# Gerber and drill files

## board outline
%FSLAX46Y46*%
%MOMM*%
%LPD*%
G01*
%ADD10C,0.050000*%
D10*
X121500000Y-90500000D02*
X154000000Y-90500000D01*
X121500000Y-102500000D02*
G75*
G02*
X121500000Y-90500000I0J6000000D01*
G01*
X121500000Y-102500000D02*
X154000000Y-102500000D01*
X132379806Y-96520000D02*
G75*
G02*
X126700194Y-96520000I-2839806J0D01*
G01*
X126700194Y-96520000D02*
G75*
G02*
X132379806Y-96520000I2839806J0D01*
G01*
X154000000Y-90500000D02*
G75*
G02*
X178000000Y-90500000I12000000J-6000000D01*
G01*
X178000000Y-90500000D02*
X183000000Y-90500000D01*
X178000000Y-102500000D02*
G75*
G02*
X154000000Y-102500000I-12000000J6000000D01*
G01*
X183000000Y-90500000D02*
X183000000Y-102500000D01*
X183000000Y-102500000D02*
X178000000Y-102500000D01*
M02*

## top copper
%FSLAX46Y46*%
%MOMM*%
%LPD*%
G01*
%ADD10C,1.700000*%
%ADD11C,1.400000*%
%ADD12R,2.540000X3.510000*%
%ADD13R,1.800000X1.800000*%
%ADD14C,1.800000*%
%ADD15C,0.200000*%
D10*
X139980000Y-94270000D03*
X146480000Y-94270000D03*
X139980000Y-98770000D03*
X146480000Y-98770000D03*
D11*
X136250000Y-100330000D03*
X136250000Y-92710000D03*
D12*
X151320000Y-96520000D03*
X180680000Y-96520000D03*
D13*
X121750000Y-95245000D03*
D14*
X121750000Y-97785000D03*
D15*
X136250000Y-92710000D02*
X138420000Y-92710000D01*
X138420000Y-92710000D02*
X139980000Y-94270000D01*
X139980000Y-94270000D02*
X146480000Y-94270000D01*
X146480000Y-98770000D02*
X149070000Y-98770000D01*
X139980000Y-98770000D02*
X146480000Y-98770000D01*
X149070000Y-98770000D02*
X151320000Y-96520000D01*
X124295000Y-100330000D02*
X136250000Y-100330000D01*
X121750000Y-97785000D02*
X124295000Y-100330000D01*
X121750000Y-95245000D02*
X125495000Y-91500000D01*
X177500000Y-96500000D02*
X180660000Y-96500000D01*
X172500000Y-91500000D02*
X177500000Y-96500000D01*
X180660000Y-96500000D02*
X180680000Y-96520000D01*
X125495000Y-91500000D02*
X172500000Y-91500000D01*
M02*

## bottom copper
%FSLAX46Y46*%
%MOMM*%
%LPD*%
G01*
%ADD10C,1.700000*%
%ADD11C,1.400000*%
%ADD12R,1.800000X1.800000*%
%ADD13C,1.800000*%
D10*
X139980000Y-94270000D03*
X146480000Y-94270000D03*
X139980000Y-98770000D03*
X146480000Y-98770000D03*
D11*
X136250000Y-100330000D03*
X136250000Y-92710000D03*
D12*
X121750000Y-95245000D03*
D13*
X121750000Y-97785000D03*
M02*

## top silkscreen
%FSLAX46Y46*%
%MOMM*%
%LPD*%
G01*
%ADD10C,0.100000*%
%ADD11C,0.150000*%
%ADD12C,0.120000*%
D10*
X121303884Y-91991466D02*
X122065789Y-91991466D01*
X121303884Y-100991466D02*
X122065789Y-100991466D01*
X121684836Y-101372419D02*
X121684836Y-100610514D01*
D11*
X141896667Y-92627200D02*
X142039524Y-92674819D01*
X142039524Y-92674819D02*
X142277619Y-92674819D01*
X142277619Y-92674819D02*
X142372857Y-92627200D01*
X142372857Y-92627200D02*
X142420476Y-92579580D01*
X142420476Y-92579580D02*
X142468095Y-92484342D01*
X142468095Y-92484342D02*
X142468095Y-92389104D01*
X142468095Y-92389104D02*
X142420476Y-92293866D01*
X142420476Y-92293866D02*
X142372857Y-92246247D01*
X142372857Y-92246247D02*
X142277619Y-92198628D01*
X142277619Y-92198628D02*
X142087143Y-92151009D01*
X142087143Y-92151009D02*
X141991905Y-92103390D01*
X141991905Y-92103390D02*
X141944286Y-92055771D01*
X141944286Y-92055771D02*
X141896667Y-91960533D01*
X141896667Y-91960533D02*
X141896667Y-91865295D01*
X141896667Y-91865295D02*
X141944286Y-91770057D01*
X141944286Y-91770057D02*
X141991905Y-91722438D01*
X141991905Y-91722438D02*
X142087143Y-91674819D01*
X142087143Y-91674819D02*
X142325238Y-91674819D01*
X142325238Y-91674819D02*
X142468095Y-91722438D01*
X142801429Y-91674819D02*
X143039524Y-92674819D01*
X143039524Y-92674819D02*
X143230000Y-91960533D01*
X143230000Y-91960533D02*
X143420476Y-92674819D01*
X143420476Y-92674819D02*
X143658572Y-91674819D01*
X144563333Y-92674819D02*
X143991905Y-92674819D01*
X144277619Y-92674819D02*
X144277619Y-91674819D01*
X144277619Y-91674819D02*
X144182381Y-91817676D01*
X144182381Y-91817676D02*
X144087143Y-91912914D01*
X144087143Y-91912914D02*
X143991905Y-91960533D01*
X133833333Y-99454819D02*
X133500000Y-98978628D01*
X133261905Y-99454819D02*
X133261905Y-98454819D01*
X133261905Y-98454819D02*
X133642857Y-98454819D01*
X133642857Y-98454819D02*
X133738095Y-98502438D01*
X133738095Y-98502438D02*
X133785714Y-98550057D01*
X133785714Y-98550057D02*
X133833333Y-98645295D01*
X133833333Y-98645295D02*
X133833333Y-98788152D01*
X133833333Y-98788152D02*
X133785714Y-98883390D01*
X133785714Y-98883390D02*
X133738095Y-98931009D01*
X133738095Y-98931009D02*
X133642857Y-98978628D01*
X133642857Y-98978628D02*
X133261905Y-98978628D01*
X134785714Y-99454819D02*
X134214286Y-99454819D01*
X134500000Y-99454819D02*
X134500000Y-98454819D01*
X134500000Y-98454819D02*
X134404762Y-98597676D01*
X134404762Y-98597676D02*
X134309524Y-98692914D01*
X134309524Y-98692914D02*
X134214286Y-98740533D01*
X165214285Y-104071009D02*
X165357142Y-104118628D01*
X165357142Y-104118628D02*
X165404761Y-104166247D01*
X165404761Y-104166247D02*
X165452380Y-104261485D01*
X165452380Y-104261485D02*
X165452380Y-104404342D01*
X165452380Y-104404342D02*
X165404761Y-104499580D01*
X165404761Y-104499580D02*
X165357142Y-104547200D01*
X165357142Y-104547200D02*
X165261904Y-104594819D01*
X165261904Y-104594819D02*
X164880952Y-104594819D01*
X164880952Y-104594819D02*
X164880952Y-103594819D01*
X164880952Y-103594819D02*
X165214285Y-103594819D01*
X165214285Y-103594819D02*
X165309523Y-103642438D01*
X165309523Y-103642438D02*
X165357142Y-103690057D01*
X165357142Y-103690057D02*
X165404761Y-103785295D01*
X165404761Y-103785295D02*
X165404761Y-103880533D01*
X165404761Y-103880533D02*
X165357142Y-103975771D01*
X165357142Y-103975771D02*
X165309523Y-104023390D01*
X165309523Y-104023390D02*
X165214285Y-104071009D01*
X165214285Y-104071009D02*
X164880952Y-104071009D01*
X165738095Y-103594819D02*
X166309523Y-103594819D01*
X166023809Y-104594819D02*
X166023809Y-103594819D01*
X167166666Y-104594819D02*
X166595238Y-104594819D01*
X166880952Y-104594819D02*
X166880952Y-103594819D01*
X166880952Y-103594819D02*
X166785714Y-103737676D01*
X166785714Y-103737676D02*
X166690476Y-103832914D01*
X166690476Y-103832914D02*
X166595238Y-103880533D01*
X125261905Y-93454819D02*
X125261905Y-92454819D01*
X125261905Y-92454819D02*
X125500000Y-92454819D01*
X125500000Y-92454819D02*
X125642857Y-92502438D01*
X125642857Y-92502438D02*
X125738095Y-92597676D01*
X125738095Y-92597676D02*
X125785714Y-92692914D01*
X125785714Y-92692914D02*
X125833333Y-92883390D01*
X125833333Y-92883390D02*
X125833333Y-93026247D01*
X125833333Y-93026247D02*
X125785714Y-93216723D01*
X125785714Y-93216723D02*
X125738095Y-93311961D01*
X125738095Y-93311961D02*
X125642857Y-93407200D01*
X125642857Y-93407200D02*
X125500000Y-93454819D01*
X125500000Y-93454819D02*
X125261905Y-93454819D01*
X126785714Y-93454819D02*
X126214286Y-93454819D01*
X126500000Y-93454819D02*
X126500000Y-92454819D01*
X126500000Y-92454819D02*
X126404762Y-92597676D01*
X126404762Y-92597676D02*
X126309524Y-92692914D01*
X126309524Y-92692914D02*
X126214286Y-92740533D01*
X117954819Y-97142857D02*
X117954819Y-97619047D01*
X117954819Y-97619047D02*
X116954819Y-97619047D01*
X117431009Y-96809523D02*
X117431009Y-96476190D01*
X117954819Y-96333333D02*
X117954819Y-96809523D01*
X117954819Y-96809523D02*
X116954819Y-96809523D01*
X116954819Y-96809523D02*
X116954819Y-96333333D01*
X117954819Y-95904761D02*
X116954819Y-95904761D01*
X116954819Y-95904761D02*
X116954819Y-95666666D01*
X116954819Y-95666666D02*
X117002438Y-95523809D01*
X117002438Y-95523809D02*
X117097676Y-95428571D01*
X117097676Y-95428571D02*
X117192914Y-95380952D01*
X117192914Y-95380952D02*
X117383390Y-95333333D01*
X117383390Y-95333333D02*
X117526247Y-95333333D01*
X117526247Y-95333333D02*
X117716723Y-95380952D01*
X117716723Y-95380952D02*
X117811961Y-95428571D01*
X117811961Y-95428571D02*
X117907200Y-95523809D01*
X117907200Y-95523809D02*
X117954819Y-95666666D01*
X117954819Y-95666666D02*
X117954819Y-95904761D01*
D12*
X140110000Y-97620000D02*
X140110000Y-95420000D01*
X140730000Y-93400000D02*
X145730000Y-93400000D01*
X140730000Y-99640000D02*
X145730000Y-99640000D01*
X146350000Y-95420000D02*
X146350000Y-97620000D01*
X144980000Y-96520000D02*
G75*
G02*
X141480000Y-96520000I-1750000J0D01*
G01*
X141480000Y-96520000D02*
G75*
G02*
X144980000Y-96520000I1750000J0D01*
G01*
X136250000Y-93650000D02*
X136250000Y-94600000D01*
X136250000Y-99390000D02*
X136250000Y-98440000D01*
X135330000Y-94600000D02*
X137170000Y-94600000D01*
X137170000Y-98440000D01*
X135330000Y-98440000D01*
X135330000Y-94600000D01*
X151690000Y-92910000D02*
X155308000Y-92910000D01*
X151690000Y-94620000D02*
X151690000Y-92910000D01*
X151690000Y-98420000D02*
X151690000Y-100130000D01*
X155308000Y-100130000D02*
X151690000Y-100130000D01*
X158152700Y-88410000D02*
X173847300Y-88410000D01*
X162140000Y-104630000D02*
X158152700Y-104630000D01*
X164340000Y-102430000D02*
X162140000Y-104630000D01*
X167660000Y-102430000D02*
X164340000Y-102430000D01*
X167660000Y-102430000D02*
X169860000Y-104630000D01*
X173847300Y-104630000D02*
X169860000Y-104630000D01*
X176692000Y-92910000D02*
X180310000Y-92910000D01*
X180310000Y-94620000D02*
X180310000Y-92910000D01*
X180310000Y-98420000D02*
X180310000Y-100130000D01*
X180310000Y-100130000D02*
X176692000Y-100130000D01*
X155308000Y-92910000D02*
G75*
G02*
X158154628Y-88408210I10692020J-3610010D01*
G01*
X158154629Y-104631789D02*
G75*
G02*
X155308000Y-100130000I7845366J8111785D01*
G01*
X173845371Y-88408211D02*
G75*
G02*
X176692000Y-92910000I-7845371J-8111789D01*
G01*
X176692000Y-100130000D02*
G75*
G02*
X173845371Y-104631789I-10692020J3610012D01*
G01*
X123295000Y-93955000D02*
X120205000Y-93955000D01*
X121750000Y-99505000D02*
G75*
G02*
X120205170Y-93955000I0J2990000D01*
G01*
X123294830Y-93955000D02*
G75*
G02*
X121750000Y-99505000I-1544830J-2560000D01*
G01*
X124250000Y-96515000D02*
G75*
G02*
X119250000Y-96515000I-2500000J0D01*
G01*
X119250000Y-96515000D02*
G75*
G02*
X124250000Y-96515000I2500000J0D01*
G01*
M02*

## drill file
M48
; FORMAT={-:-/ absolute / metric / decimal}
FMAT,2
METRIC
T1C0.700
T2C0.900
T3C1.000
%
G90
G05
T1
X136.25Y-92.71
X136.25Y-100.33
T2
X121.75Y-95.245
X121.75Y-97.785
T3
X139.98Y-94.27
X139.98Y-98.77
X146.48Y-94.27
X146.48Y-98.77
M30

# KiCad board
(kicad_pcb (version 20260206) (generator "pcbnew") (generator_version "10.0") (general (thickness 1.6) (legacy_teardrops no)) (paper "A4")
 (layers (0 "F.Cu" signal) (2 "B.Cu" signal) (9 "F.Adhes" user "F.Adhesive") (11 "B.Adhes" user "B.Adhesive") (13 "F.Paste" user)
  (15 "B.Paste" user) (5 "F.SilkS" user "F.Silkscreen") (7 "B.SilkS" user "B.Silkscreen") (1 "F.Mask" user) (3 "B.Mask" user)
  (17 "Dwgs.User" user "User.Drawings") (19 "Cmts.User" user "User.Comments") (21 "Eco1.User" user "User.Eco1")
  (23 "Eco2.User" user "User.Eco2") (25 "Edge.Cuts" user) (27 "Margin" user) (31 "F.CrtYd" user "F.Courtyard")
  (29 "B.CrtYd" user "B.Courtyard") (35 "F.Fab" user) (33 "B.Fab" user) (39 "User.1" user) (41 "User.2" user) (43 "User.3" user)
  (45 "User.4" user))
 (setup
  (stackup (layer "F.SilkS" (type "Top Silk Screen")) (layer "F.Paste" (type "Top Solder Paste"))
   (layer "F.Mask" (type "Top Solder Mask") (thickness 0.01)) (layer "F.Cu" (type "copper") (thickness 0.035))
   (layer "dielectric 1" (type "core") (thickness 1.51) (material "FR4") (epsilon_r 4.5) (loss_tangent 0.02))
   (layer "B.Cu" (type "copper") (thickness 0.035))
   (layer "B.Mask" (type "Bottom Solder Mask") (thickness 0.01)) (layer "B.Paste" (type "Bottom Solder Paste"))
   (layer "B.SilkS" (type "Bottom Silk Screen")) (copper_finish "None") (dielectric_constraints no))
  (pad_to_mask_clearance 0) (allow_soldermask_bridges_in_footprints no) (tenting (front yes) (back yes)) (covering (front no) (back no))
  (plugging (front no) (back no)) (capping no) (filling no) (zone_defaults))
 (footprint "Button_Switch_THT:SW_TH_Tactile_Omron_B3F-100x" (layer "F.Cu") (at 139.98 94.27)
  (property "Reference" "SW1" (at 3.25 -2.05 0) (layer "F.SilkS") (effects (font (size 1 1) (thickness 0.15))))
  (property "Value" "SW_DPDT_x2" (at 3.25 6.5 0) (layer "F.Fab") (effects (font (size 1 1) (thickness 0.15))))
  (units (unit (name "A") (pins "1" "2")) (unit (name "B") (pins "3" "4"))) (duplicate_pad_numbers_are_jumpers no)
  (fp_line (start 0.13 3.35) (end 0.13 1.15) (stroke (width 0.12) (type solid)) (layer "F.SilkS"))
  (fp_line (start 0.75 -0.87) (end 5.75 -0.87) (stroke (width 0.12) (type solid)) (layer "F.SilkS"))
  (fp_line (start 0.75 5.37) (end 5.75 5.37) (stroke (width 0.12) (type solid)) (layer "F.SilkS"))
  (fp_line (start 6.37 1.15) (end 6.37 3.35) (stroke (width 0.12) (type solid)) (layer "F.SilkS"))
  (fp_circle (center 3.25 2.25) (end 5 2.25) (stroke (width 0.12) (type solid)) (fill no) (layer "F.SilkS"))
  (pad "1" thru_hole circle (at 0 0) (size 1.7 1.7) (drill 1) (layers "*.Cu" "*.Mask") (remove_unused_layers no) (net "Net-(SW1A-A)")
   (thermal_bridge_angle 90))
  (pad "1" thru_hole circle (at 6.5 0) (size 1.7 1.7) (drill 1) (layers "*.Cu" "*.Mask") (remove_unused_layers no) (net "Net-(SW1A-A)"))
  (pad "2" thru_hole circle (at 0 4.5) (size 1.7 1.7) (drill 1) (layers "*.Cu" "*.Mask") (remove_unused_layers no) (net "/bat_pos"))
  (pad "2" thru_hole circle (at 6.5 4.5) (size 1.7 1.7) (drill 1) (layers "*.Cu" "*.Mask") (remove_unused_layers no) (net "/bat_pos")))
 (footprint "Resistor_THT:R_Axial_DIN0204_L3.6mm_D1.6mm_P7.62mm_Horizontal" (layer "F.Cu") (at 136.25 100.33 90)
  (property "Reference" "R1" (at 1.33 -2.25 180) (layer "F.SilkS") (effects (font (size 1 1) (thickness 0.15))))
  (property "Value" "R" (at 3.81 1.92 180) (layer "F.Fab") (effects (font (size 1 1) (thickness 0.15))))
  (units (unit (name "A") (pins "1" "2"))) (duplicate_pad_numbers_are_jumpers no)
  (fp_line (start 6.68 0) (end 5.73 0) (stroke (width 0.12) (type solid)) (layer "F.SilkS"))
  (fp_line (start 0.94 0) (end 1.89 0) (stroke (width 0.12) (type solid)) (layer "F.SilkS"))
  (fp_rect (start 1.89 -0.92) (end 5.73 0.92) (stroke (width 0.12) (type solid)) (fill no) (layer "F.SilkS"))
  (pad "1" thru_hole circle (at 0 0 90) (size 1.4 1.4) (drill 0.7) (layers "*.Cu" "*.Mask") (remove_unused_layers no) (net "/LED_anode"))
  (pad "2" thru_hole circle (at 7.62 0 90) (size 1.4 1.4) (drill 0.7) (layers "*.Cu" "*.Mask") (remove_unused_layers no)
   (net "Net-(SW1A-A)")))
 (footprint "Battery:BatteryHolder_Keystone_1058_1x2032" (layer "F.Cu") (at 166 96.52)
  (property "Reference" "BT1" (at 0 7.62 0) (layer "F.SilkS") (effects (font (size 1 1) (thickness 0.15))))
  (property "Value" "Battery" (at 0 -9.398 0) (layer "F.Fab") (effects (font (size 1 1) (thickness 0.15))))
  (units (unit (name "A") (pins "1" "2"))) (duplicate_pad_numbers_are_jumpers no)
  (fp_line (start -14.31 -3.61) (end -10.692 -3.61) (stroke (width 0.12) (type solid)) (layer "F.SilkS"))
  (fp_line (start -14.31 -1.9) (end -14.31 -3.61) (stroke (width 0.12) (type solid)) (layer "F.SilkS"))
  (fp_line (start -14.31 1.9) (end -14.31 3.61) (stroke (width 0.12) (type solid)) (layer "F.SilkS"))
  (fp_line (start -10.692 3.61) (end -14.31 3.61) (stroke (width 0.12) (type solid)) (layer "F.SilkS"))
  (fp_line (start -7.8473 -8.11) (end 7.8473 -8.11) (stroke (width 0.12) (type solid)) (layer "F.SilkS"))
  (fp_line (start -3.86 8.11) (end -7.8473 8.11) (stroke (width 0.12) (type solid)) (layer "F.SilkS"))
  (fp_line (start -1.66 5.91) (end -3.86 8.11) (stroke (width 0.12) (type solid)) (layer "F.SilkS"))
  (fp_line (start 1.66 5.91) (end -1.66 5.91) (stroke (width 0.12) (type solid)) (layer "F.SilkS"))
  (fp_line (start 1.66 5.91) (end 3.86 8.11) (stroke (width 0.12) (type solid)) (layer "F.SilkS"))
  (fp_line (start 7.8473 8.11) (end 3.86 8.11) (stroke (width 0.12) (type solid)) (layer "F.SilkS"))
  (fp_line (start 10.692 -3.61) (end 14.31 -3.61) (stroke (width 0.12) (type solid)) (layer "F.SilkS"))
  (fp_line (start 14.31 -1.9) (end 14.31 -3.61) (stroke (width 0.12) (type solid)) (layer "F.SilkS"))
  (fp_line (start 14.31 1.9) (end 14.31 3.61) (stroke (width 0.12) (type solid)) (layer "F.SilkS"))
  (fp_line (start 14.31 3.61) (end 10.692 3.61) (stroke (width 0.12) (type solid)) (layer "F.SilkS"))
  (fp_arc (start -10.692 -3.61) (mid -9.538084 -6.031244) (end -7.845371 -8.111789) (stroke (width 0.12) (type solid)) (layer "F.SilkS"))
  (fp_arc (start -7.845371 8.111789) (mid -9.538085 6.031244) (end -10.692 3.61) (stroke (width 0.12) (type solid)) (layer "F.SilkS"))
  (fp_arc (start 7.845371 -8.111789) (mid 9.538085 -6.031244) (end 10.692 -3.61) (stroke (width 0.12) (type solid)) (layer "F.SilkS"))
  (fp_arc (start 10.692 3.61) (mid 9.538084 6.031244) (end 7.845371 8.111789) (stroke (width 0.12) (type solid)) (layer "F.SilkS"))
  (pad "1" smd rect (at -14.68 0) (size 2.54 3.51) (layers "F.Cu" "F.Mask" "F.Paste") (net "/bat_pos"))
  (pad "2" smd rect (at 14.68 0) (size 2.54 3.51) (layers "F.Cu" "F.Mask" "F.Paste") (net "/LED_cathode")))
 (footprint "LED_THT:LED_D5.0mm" (layer "F.Cu") (at 121.75 95.245 -90)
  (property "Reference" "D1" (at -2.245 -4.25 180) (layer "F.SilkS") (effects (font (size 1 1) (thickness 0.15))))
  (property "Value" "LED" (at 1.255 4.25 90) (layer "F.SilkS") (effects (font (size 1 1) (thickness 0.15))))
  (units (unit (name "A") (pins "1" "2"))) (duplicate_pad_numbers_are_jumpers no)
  (fp_line (start -1.29 -1.545) (end -1.29 1.545) (stroke (width 0.12) (type solid)) (layer "F.SilkS"))
  (fp_arc (start 4.26 0) (mid 2.071779 2.880495) (end -1.29 1.54483) (stroke (width 0.12) (type solid)) (layer "F.SilkS"))
  (fp_arc (start -1.29 -1.54483) (mid 2.071779 -2.880495) (end 4.26 0) (stroke (width 0.12) (type solid)) (layer "F.SilkS"))
  (fp_circle (center 1.27 0) (end 3.77 0) (stroke (width 0.12) (type solid)) (fill no) (layer "F.SilkS"))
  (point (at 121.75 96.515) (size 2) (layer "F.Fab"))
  (pad "1" thru_hole rect (at 0 0 270) (size 1.8 1.8) (drill 0.9) (layers "*.Cu" "*.Mask") (remove_unused_layers no) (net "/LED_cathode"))
  (pad "2" thru_hole circle (at 2.54 0 270) (size 1.8 1.8) (drill 0.9) (layers "*.Cu" "*.Mask") (remove_unused_layers no) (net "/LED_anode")))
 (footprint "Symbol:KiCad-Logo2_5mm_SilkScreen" (layer "B.Cu") (at 166 92.5 180)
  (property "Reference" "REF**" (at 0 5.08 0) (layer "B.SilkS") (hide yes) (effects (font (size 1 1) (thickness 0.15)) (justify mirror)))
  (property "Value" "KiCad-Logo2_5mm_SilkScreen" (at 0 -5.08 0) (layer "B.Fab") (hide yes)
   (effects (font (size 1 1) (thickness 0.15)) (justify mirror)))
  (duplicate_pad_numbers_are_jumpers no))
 (gr_line (start 121.5 90.5) (end 154 90.5) (stroke (width 0.05) (type default)) (locked yes) (layer "Edge.Cuts"))
 (gr_arc (start 121.5 102.5) (mid 115.5 96.5) (end 121.5 90.5) (stroke (width 0.05) (type default)) (locked yes) (layer "Edge.Cuts"))
 (gr_line (start 121.5 102.5) (end 154 102.5) (stroke (width 0.05) (type default)) (locked yes) (layer "Edge.Cuts"))
 (gr_circle (center 129.54 96.52) (end 130.81 99.06) (stroke (width 0.05) (type default)) (fill no) (locked yes) (layer "Edge.Cuts"))
 (gr_arc (start 154 90.5) (mid 166 83.083592) (end 178 90.5) (stroke (width 0.05) (type default)) (locked yes) (layer "Edge.Cuts"))
 (gr_line (start 178 90.5) (end 183 90.5) (stroke (width 0.05) (type default)) (locked yes) (layer "Edge.Cuts"))
 (gr_arc (start 178 102.5) (mid 166 109.916408) (end 154 102.5) (stroke (width 0.05) (type default)) (locked yes) (layer "Edge.Cuts"))
 (gr_line (start 183 90.5) (end 183 102.5) (stroke (width 0.05) (type default)) (locked yes) (layer "Edge.Cuts"))
 (gr_line (start 183 102.5) (end 178 102.5) (stroke (width 0.05) (type default)) (locked yes) (layer "Edge.Cuts"))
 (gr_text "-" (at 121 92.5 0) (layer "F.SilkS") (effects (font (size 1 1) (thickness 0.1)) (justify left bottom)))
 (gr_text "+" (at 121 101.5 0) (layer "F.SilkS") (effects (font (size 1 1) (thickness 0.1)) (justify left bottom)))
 (segment (start 136.25 92.71) (end 138.42 92.71) (width 0.2) (layer "F.Cu") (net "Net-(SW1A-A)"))
 (segment (start 138.42 92.71) (end 139.98 94.27) (width 0.2) (layer "F.Cu") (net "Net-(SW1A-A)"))
 (segment (start 139.98 94.27) (end 146.48 94.27) (width 0.2) (layer "F.Cu") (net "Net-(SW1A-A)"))
 (segment (start 146.48 98.77) (end 149.07 98.77) (width 0.2) (layer "F.Cu") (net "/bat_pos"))
 (segment (start 139.98 98.77) (end 146.48 98.77) (width 0.2) (layer "F.Cu") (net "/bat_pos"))
 (segment (start 149.07 98.77) (end 151.32 96.52) (width 0.2) (layer "F.Cu") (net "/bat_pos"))
 (segment (start 124.295 100.33) (end 136.25 100.33) (width 0.2) (layer "F.Cu") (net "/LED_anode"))
 (segment (start 121.75 97.785) (end 124.295 100.33) (width 0.2) (layer "F.Cu") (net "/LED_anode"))
 (segment (start 121.75 95.245) (end 125.495 91.5) (width 0.2) (layer "F.Cu") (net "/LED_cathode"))
 (segment (start 177.5 96.5) (end 180.66 96.5) (width 0.2) (layer "F.Cu") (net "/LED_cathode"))
 (segment (start 172.5 91.5) (end 177.5 96.5) (width 0.2) (layer "F.Cu") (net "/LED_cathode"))
 (segment (start 180.66 96.5) (end 180.68 96.52) (width 0.2) (layer "F.Cu") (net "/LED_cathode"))
 (segment (start 125.495 91.5) (end 172.5 91.5) (width 0.2) (layer "F.Cu") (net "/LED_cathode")))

